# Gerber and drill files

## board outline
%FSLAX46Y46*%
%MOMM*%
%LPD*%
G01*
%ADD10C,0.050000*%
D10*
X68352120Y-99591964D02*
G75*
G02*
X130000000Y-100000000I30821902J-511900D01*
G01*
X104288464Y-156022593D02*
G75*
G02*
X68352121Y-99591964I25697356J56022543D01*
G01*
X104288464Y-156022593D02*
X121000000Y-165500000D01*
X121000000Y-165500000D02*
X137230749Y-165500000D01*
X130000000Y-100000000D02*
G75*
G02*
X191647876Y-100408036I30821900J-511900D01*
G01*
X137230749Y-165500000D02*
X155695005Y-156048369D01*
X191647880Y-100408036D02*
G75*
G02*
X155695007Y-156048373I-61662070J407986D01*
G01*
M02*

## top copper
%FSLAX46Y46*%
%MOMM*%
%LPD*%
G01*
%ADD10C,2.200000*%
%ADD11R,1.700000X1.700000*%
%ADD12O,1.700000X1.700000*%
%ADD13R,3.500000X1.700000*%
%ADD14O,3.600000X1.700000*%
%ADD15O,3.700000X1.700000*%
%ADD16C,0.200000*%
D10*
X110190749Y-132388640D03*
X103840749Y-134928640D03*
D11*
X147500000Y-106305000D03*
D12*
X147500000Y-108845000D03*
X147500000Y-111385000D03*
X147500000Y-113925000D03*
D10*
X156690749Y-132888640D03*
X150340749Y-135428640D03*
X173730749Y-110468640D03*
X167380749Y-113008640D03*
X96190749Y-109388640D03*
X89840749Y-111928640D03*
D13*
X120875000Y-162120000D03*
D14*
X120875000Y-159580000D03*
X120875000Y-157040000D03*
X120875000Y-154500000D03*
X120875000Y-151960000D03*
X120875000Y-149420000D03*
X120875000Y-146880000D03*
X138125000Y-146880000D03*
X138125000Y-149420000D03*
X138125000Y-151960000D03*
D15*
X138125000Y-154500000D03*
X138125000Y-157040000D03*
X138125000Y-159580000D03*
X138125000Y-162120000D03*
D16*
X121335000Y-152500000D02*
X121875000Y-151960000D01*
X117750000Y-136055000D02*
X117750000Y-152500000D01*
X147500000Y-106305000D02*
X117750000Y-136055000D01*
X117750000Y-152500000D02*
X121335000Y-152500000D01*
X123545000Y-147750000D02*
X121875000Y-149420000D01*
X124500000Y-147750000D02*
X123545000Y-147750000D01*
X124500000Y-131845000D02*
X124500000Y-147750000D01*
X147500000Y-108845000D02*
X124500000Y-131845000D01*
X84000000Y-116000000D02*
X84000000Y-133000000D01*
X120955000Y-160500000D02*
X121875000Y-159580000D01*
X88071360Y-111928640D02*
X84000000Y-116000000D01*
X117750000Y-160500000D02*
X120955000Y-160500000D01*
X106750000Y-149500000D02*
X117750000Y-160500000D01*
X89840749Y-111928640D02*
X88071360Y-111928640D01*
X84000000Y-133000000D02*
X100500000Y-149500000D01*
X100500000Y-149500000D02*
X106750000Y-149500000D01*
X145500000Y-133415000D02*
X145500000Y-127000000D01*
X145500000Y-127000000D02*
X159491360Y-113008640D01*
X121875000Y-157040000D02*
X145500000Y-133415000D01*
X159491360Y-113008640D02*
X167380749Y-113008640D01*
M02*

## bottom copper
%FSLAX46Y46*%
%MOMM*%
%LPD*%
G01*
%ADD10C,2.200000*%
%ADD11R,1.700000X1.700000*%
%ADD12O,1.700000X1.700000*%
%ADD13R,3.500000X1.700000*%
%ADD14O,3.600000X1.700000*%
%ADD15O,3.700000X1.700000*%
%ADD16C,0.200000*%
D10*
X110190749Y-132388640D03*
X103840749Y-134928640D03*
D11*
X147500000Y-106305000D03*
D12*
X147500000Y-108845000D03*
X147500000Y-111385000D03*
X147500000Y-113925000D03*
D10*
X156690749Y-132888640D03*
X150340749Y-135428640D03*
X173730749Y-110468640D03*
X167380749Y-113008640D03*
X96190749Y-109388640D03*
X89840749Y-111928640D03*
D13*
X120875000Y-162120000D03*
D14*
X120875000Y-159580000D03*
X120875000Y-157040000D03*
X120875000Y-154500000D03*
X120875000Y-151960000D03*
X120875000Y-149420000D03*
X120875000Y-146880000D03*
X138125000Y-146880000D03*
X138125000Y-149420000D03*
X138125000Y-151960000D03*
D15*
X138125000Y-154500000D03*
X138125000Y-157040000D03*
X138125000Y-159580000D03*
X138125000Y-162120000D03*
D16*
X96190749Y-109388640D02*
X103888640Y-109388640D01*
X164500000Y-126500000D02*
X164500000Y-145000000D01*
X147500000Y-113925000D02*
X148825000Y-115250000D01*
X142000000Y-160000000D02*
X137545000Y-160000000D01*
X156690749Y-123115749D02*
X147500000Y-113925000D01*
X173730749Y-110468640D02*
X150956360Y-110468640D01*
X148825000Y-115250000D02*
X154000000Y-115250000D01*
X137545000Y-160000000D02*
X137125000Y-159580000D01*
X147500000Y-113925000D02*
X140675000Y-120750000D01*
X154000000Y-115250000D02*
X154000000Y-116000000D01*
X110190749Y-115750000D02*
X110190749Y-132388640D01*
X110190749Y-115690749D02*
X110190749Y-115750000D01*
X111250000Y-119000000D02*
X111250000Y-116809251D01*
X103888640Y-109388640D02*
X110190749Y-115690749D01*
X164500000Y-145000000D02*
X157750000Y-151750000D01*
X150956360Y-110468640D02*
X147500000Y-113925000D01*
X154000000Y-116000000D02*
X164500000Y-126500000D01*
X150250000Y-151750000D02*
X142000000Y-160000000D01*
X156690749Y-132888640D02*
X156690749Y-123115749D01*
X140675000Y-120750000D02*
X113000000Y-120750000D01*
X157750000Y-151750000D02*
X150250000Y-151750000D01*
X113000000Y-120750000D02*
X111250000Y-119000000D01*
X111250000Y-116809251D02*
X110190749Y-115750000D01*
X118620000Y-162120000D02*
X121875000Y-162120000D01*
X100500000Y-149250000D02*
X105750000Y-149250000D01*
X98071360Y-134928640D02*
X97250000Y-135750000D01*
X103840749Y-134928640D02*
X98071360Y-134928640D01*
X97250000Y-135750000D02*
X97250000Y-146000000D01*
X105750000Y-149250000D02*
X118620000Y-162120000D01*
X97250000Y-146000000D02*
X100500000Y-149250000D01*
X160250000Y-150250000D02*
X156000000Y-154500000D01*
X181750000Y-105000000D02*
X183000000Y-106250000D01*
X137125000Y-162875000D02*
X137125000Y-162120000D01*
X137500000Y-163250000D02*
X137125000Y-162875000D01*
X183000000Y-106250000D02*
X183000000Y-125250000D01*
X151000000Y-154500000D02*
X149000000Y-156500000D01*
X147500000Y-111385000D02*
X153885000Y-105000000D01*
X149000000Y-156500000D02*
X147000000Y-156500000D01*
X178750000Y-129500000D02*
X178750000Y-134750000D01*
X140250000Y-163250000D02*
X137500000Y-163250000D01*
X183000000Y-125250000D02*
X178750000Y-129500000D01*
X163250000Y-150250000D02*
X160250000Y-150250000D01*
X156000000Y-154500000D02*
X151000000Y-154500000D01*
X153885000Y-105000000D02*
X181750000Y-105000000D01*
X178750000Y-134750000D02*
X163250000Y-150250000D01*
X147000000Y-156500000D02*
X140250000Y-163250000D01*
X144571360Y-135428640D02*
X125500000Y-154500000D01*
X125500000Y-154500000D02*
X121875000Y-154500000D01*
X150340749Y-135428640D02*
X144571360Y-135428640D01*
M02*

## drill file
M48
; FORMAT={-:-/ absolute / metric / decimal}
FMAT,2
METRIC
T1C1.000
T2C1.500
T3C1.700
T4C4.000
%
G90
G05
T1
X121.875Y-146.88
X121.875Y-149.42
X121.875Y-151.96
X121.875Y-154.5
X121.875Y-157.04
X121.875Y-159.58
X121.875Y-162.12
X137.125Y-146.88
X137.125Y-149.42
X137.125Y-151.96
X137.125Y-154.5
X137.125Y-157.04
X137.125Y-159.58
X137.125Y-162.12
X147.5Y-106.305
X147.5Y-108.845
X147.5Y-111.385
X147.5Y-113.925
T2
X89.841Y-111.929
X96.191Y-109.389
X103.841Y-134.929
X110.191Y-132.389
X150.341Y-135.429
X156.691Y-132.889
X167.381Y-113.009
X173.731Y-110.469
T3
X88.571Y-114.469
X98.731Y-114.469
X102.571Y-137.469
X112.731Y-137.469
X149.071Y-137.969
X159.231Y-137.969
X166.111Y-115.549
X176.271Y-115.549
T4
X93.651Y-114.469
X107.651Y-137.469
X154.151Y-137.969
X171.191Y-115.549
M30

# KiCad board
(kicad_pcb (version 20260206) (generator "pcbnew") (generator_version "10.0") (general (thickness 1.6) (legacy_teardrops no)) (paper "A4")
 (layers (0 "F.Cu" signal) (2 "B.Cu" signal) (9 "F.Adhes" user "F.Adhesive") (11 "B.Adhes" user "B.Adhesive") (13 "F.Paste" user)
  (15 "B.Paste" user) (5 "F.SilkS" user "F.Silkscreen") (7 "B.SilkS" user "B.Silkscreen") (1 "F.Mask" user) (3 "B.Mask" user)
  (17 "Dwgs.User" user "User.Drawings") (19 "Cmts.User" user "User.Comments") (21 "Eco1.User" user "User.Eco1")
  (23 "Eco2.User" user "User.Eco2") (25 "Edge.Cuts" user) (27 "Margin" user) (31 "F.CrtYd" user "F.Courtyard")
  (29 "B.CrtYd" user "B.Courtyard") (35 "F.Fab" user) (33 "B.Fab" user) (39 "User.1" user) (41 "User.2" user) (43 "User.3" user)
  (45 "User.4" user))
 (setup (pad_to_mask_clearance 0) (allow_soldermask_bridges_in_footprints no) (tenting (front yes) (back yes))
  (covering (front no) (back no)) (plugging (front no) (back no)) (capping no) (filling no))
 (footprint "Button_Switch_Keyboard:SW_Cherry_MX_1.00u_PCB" (layer "F.Cu") (at 110.190749 132.38864)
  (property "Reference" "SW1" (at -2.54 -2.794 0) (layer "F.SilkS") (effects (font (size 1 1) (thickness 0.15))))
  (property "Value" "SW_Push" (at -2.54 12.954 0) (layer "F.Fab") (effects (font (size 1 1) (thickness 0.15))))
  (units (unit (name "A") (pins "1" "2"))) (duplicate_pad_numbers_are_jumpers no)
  (pad "" np_thru_hole circle (at -7.62 5.08) (size 1.7 1.7) (drill 1.7) (layers "*.Cu" "*.Mask"))
  (pad "" np_thru_hole circle (at -2.54 5.08) (size 4 4) (drill 4) (layers "*.Cu" "*.Mask"))
  (pad "" np_thru_hole circle (at 2.54 5.08) (size 1.7 1.7) (drill 1.7) (layers "*.Cu" "*.Mask"))
  (pad "1" thru_hole circle (at 0 0) (size 2.2 2.2) (drill 1.5) (layers "*.Cu" "*.Mask") (remove_unused_layers no) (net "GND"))
  (pad "2" thru_hole circle (at -6.35 2.54) (size 2.2 2.2) (drill 1.5) (layers "*.Cu" "*.Mask") (remove_unused_layers no)
   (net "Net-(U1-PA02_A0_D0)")))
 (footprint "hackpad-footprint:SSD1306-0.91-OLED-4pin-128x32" (layer "F.Cu") (at 111 104.115)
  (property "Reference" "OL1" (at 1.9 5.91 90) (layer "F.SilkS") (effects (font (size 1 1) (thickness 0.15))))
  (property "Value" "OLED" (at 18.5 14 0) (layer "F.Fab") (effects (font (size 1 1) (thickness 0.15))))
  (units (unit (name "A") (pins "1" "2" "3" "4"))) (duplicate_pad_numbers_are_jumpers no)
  (pad "1" thru_hole rect (at 36.5 2.19) (size 1.7 1.7) (drill 1) (layers "*.Cu" "*.Mask") (remove_unused_layers no) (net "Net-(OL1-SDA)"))
  (pad "2" thru_hole oval (at 36.5 4.73) (size 1.7 1.7) (drill 1) (layers "*.Cu" "*.Mask") (remove_unused_layers no) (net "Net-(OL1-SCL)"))
  (pad "3" thru_hole oval (at 36.5 7.27) (size 1.7 1.7) (drill 1) (layers "*.Cu" "*.Mask") (remove_unused_layers no) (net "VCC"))
  (pad "4" thru_hole oval (at 36.5 9.81) (size 1.7 1.7) (drill 1) (layers "*.Cu" "*.Mask") (remove_unused_layers no) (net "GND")))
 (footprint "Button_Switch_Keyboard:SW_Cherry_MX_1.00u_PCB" (layer "F.Cu") (at 156.690749 132.88864)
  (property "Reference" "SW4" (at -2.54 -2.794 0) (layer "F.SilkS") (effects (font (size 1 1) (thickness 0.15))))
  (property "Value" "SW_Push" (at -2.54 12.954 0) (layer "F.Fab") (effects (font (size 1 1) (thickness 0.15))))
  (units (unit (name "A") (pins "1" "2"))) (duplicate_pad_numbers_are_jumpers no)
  (pad "" np_thru_hole circle (at -7.62 5.08) (size 1.7 1.7) (drill 1.7) (layers "*.Cu" "*.Mask"))
  (pad "" np_thru_hole circle (at -2.54 5.08) (size 4 4) (drill 4) (layers "*.Cu" "*.Mask"))
  (pad "" np_thru_hole circle (at 2.54 5.08) (size 1.7 1.7) (drill 1.7) (layers "*.Cu" "*.Mask"))
  (pad "1" thru_hole circle (at 0 0) (size 2.2 2.2) (drill 1.5) (layers "*.Cu" "*.Mask") (remove_unused_layers no) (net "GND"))
  (pad "2" thru_hole circle (at -6.35 2.54) (size 2.2 2.2) (drill 1.5) (layers "*.Cu" "*.Mask") (remove_unused_layers no)
   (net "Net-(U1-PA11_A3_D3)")))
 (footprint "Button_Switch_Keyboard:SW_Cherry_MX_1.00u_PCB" (layer "F.Cu") (at 173.730749 110.46864)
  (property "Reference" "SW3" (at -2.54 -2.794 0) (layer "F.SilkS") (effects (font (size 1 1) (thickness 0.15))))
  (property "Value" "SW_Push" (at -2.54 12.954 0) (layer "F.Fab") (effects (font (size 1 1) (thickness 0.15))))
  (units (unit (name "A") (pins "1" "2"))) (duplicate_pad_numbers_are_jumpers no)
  (pad "" np_thru_hole circle (at -7.62 5.08) (size 1.7 1.7) (drill 1.7) (layers "*.Cu" "*.Mask"))
  (pad "" np_thru_hole circle (at -2.54 5.08) (size 4 4) (drill 4) (layers "*.Cu" "*.Mask"))
  (pad "" np_thru_hole circle (at 2.54 5.08) (size 1.7 1.7) (drill 1.7) (layers "*.Cu" "*.Mask"))
  (pad "1" thru_hole circle (at 0 0) (size 2.2 2.2) (drill 1.5) (layers "*.Cu" "*.Mask") (remove_unused_layers no) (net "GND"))
  (pad "2" thru_hole circle (at -6.35 2.54) (size 2.2 2.2) (drill 1.5) (layers "*.Cu" "*.Mask") (remove_unused_layers no)
   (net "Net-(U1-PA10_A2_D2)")))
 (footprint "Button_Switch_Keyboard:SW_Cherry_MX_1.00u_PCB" (layer "F.Cu") (at 96.190749 109.38864)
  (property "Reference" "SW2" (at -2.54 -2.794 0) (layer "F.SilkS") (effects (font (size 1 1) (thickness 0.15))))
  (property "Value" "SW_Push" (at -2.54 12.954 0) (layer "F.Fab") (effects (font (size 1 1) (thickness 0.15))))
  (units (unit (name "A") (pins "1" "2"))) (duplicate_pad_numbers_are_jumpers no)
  (pad "" np_thru_hole circle (at -7.62 5.08) (size 1.7 1.7) (drill 1.7) (layers "*.Cu" "*.Mask"))
  (pad "" np_thru_hole circle (at -2.54 5.08) (size 4 4) (drill 4) (layers "*.Cu" "*.Mask"))
  (pad "" np_thru_hole circle (at 2.54 5.08) (size 1.7 1.7) (drill 1.7) (layers "*.Cu" "*.Mask"))
  (pad "1" thru_hole circle (at 0 0) (size 2.2 2.2) (drill 1.5) (layers "*.Cu" "*.Mask") (remove_unused_layers no) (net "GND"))
  (pad "2" thru_hole circle (at -6.35 2.54) (size 2.2 2.2) (drill 1.5) (layers "*.Cu" "*.Mask") (remove_unused_layers no)
   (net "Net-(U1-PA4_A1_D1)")))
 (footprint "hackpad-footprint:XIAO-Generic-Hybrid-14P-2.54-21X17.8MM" (layer "B.Cu") (at 129.5 154.5)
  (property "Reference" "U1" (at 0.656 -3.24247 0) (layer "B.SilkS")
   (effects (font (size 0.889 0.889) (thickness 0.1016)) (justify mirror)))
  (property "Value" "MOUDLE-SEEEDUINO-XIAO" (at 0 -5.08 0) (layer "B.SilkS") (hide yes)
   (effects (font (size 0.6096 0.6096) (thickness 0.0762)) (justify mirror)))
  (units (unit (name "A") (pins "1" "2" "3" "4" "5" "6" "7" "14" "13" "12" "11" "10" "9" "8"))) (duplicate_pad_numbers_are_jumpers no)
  (pad "1" thru_hole rect (at -7.625 7.62) (size 3.5 1.7) (drill 1 (offset -1 0)) (layers "*.Cu" "*.Mask") (remove_unused_layers no)
   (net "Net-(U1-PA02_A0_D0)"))
  (pad "2" thru_hole oval (at -7.625 5.08) (size 3.6 1.7) (drill 1 (offset -1 0)) (layers "*.Cu" "*.Mask") (remove_unused_layers no)
   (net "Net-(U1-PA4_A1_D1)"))
  (pad "3" thru_hole oval (at -7.625 2.54) (size 3.6 1.7) (drill 1 (offset -1 0)) (layers "*.Cu" "*.Mask") (remove_unused_layers no)
   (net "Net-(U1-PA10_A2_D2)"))
  (pad "4" thru_hole oval (at -7.625 0) (size 3.6 1.7) (drill 1 (offset -1 0)) (layers "*.Cu" "*.Mask") (remove_unused_layers no)
   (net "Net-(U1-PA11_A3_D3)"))
  (pad "5" thru_hole oval (at -7.625 -2.54) (size 3.6 1.7) (drill 1 (offset -1 0)) (layers "*.Cu" "*.Mask") (remove_unused_layers no)
   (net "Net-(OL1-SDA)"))
  (pad "6" thru_hole oval (at -7.625 -5.08 180) (size 3.6 1.7) (drill 1 (offset 1 0)) (layers "*.Cu" "*.Mask") (remove_unused_layers no)
   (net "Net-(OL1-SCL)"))
  (pad "7" thru_hole oval (at -7.625 -7.62) (size 3.6 1.7) (drill 1 (offset -1 0)) (layers "*.Cu" "*.Mask") (remove_unused_layers no)
   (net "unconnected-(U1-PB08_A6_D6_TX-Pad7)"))
  (pad "8" thru_hole oval (at 7.625 -7.62) (size 3.6 1.7) (drill 1 (offset 1 0)) (layers "*.Cu" "*.Mask") (remove_unused_layers no)
   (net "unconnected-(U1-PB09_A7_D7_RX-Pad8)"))
  (pad "9" thru_hole oval (at 7.625 -5.08) (size 3.6 1.7) (drill 1 (offset 1 0)) (layers "*.Cu" "*.Mask") (remove_unused_layers no)
   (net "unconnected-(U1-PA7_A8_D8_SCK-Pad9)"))
  (pad "10" thru_hole oval (at 7.625 -2.54) (size 3.6 1.7) (drill 1 (offset 1 0)) (layers "*.Cu" "*.Mask") (remove_unused_layers no)
   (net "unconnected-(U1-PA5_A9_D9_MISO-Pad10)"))
  (pad "11" thru_hole oval (at 7.625 0) (size 3.7 1.7) (drill 1 (offset 1 0)) (layers "*.Cu" "*.Mask") (remove_unused_layers no)
   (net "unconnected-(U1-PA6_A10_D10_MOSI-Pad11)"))
  (pad "12" thru_hole oval (at 7.625 2.54) (size 3.7 1.7) (drill 1 (offset 1 0)) (layers "*.Cu" "*.Mask") (remove_unused_layers no)
   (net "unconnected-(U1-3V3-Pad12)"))
  (pad "13" thru_hole oval (at 7.625 5.08) (size 3.7 1.7) (drill 1 (offset 1 0)) (layers "*.Cu" "*.Mask") (remove_unused_layers no)
   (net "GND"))
  (pad "14" thru_hole oval (at 7.625 7.62) (size 3.7 1.7) (drill 1 (offset 1 0)) (layers "*.Cu" "*.Mask") (remove_unused_layers no)
   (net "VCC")))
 (gr_arc (start 68.35212 99.591964) (mid 99.37805 69.278386) (end 130 100) (stroke (width 0.05) (type default)) (layer "Edge.Cuts"))
 (gr_arc (start 104.288464 156.022593) (mid 77.99753 133.107408) (end 68.35212 99.591964) (stroke (width 0.05) (type default))
  (layer "Edge.Cuts"))
 (gr_line (start 104.288464 156.022593) (end 121 165.5) (stroke (width 0.05) (type default)) (layer "Edge.Cuts"))
 (gr_line (start 121 165.5) (end 137.230749 165.5) (stroke (width 0.05) (type default)) (layer "Edge.Cuts"))
 (gr_arc (start 130 100) (mid 161.02593 69.686422) (end 191.64788 100.408036) (stroke (width 0.05) (type default)) (layer "Edge.Cuts"))
 (gr_line (start 137.230749 165.5) (end 155.695005 156.048369) (stroke (width 0.05) (type default)) (layer "Edge.Cuts"))
 (gr_arc (start 191.64788 100.408036) (mid 181.777665 133.466165) (end 155.695005 156.048369) (stroke (width 0.05) (type default))
  (layer "Edge.Cuts"))
 (segment (start 96.190749 109.38864) (end 103.88864 109.38864) (width 0.2) (layer "B.Cu") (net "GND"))
 (segment (start 164.5 126.5) (end 164.5 145) (width 0.2) (layer "B.Cu") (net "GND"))
 (segment (start 147.5 113.925) (end 148.825 115.25) (width 0.2) (layer "B.Cu") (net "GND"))
 (segment (start 142 160) (end 137.545 160) (width 0.2) (layer "B.Cu") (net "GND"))
 (segment (start 156.690749 123.115749) (end 147.5 113.925) (width 0.2) (layer "B.Cu") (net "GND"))
 (segment (start 173.730749 110.46864) (end 150.95636 110.46864) (width 0.2) (layer "B.Cu") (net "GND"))
 (segment (start 148.825 115.25) (end 154 115.25) (width 0.2) (layer "B.Cu") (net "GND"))
 (segment (start 137.545 160) (end 137.125 159.58) (width 0.2) (layer "B.Cu") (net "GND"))
 (segment (start 147.5 113.925) (end 140.675 120.75) (width 0.2) (layer "B.Cu") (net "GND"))
 (segment (start 154 115.25) (end 154 116) (width 0.2) (layer "B.Cu") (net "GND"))
 (segment (start 110.190749 115.75) (end 110.190749 132.38864) (width 0.2) (layer "B.Cu") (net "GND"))
 (segment (start 110.190749 115.690749) (end 110.190749 115.75) (width 0.2) (layer "B.Cu") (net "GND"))
 (segment (start 111.25 119) (end 111.25 116.809251) (width 0.2) (layer "B.Cu") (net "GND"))
 (segment (start 103.88864 109.38864) (end 110.190749 115.690749) (width 0.2) (layer "B.Cu") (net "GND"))
 (segment (start 164.5 145) (end 157.75 151.75) (width 0.2) (layer "B.Cu") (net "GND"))
 (segment (start 150.95636 110.46864) (end 147.5 113.925) (width 0.2) (layer "B.Cu") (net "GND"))
 (segment (start 154 116) (end 164.5 126.5) (width 0.2) (layer "B.Cu") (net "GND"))
 (segment (start 150.25 151.75) (end 142 160) (width 0.2) (layer "B.Cu") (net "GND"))
 (segment (start 156.690749 132.88864) (end 156.690749 123.115749) (width 0.2) (layer "B.Cu") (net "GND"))
 (segment (start 140.675 120.75) (end 113 120.75) (width 0.2) (layer "B.Cu") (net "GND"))
 (segment (start 157.75 151.75) (end 150.25 151.75) (width 0.2) (layer "B.Cu") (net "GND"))
 (segment (start 113 120.75) (end 111.25 119) (width 0.2) (layer "B.Cu") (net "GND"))
 (segment (start 111.25 116.809251) (end 110.190749 115.75) (width 0.2) (layer "B.Cu") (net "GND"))
 (segment (start 118.62 162.12) (end 121.875 162.12) (width 0.2) (layer "B.Cu") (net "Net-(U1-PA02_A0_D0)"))
 (segment (start 100.5 149.25) (end 105.75 149.25) (width 0.2) (layer "B.Cu") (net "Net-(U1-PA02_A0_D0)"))
 (segment (start 98.07136 134.92864) (end 97.25 135.75) (width 0.2) (layer "B.Cu") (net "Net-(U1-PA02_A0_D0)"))
 (segment (start 103.840749 134.92864) (end 98.07136 134.92864) (width 0.2) (layer "B.Cu") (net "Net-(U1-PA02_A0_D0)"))
 (segment (start 97.25 135.75) (end 97.25 146) (width 0.2) (layer "B.Cu") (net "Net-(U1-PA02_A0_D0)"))
 (segment (start 105.75 149.25) (end 118.62 162.12) (width 0.2) (layer "B.Cu") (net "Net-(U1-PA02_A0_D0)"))
 (segment (start 97.25 146) (end 100.5 149.25) (width 0.2) (layer "B.Cu") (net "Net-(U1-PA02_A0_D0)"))
 (segment (start 121.335 152.5) (end 121.875 151.96) (width 0.2) (layer "F.Cu") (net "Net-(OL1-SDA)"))
 (segment (start 117.75 136.055) (end 117.75 152.5) (width 0.2) (layer "F.Cu") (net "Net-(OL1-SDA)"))
 (segment (start 147.5 106.305) (end 117.75 136.055) (width 0.2) (layer "F.Cu") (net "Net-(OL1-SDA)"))
 (segment (start 117.75 152.5) (end 121.335 152.5) (width 0.2) (layer "F.Cu") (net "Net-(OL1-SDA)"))
 (segment (start 123.545 147.75) (end 121.875 149.42) (width 0.2) (layer "F.Cu") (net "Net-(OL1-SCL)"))
 (segment (start 124.5 147.75) (end 123.545 147.75) (width 0.2) (layer "F.Cu") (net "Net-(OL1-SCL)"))
 (segment (start 124.5 131.845) (end 124.5 147.75) (width 0.2) (layer "F.Cu") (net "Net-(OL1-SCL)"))
 (segment (start 147.5 108.845) (end 124.5 131.845) (width 0.2) (layer "F.Cu") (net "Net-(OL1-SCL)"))
 (segment (start 160.25 150.25) (end 156 154.5) (width 0.2) (layer "B.Cu") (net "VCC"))
 (segment (start 181.75 105) (end 183 106.25) (width 0.2) (layer "B.Cu") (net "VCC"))
 (segment (start 137.125 162.875) (end 137.125 162.12) (width 0.2) (layer "B.Cu") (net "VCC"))
 (segment (start 137.5 163.25) (end 137.125 162.875) (width 0.2) (layer "B.Cu") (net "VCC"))
 (segment (start 183 106.25) (end 183 125.25) (width 0.2) (layer "B.Cu") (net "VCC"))
 (segment (start 151 154.5) (end 149 156.5) (width 0.2) (layer "B.Cu") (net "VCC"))
 (segment (start 147.5 111.385) (end 153.885 105) (width 0.2) (layer "B.Cu") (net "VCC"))
 (segment (start 149 156.5) (end 147 156.5) (width 0.2) (layer "B.Cu") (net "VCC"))
 (segment (start 178.75 129.5) (end 178.75 134.75) (width 0.2) (layer "B.Cu") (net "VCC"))
 (segment (start 140.25 163.25) (end 137.5 163.25) (width 0.2) (layer "B.Cu") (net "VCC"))
 (segment (start 183 125.25) (end 178.75 129.5) (width 0.2) (layer "B.Cu") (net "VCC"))
 (segment (start 163.25 150.25) (end 160.25 150.25) (width 0.2) (layer "B.Cu") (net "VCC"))
 (segment (start 156 154.5) (end 151 154.5) (width 0.2) (layer "B.Cu") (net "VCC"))
 (segment (start 153.885 105) (end 181.75 105) (width 0.2) (layer "B.Cu") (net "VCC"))
 (segment (start 178.75 134.75) (end 163.25 150.25) (width 0.2) (layer "B.Cu") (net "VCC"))
 (segment (start 147 156.5) (end 140.25 163.25) (width 0.2) (layer "B.Cu") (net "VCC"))
 (segment (start 84 116) (end 84 133) (width 0.2) (layer "F.Cu") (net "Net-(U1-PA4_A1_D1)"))
 (segment (start 120.955 160.5) (end 121.875 159.58) (width 0.2) (layer "F.Cu") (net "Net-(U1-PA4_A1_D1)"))
 (segment (start 88.07136 111.92864) (end 84 116) (width 0.2) (layer "F.Cu") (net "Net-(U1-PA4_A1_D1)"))
 (segment (start 117.75 160.5) (end 120.955 160.5) (width 0.2) (layer "F.Cu") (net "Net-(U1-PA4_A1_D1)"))
 (segment (start 106.75 149.5) (end 117.75 160.5) (width 0.2) (layer "F.Cu") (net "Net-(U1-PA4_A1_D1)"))
 (segment (start 89.840749 111.92864) (end 88.07136 111.92864) (width 0.2) (layer "F.Cu") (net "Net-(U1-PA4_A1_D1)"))
 (segment (start 84 133) (end 100.5 149.5) (width 0.2) (layer "F.Cu") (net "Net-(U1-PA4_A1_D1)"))
 (segment (start 100.5 149.5) (end 106.75 149.5) (width 0.2) (layer "F.Cu") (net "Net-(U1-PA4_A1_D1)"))
 (segment (start 145.5 133.415) (end 145.5 127) (width 0.2) (layer "F.Cu") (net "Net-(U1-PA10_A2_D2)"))
 (segment (start 145.5 127) (end 159.49136 113.00864) (width 0.2) (layer "F.Cu") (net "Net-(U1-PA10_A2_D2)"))
 (segment (start 121.875 157.04) (end 145.5 133.415) (width 0.2) (layer "F.Cu") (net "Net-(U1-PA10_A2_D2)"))
 (segment (start 159.49136 113.00864) (end 167.380749 113.00864) (width 0.2) (layer "F.Cu") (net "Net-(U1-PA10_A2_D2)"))
 (segment (start 144.57136 135.42864) (end 125.5 154.5) (width 0.2) (layer "B.Cu") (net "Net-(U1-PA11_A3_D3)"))
 (segment (start 125.5 154.5) (end 121.875 154.5) (width 0.2) (layer "B.Cu") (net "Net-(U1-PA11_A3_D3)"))
 (segment (start 150.340749 135.42864) (end 144.57136 135.42864) (width 0.2) (layer "B.Cu") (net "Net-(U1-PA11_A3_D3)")))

